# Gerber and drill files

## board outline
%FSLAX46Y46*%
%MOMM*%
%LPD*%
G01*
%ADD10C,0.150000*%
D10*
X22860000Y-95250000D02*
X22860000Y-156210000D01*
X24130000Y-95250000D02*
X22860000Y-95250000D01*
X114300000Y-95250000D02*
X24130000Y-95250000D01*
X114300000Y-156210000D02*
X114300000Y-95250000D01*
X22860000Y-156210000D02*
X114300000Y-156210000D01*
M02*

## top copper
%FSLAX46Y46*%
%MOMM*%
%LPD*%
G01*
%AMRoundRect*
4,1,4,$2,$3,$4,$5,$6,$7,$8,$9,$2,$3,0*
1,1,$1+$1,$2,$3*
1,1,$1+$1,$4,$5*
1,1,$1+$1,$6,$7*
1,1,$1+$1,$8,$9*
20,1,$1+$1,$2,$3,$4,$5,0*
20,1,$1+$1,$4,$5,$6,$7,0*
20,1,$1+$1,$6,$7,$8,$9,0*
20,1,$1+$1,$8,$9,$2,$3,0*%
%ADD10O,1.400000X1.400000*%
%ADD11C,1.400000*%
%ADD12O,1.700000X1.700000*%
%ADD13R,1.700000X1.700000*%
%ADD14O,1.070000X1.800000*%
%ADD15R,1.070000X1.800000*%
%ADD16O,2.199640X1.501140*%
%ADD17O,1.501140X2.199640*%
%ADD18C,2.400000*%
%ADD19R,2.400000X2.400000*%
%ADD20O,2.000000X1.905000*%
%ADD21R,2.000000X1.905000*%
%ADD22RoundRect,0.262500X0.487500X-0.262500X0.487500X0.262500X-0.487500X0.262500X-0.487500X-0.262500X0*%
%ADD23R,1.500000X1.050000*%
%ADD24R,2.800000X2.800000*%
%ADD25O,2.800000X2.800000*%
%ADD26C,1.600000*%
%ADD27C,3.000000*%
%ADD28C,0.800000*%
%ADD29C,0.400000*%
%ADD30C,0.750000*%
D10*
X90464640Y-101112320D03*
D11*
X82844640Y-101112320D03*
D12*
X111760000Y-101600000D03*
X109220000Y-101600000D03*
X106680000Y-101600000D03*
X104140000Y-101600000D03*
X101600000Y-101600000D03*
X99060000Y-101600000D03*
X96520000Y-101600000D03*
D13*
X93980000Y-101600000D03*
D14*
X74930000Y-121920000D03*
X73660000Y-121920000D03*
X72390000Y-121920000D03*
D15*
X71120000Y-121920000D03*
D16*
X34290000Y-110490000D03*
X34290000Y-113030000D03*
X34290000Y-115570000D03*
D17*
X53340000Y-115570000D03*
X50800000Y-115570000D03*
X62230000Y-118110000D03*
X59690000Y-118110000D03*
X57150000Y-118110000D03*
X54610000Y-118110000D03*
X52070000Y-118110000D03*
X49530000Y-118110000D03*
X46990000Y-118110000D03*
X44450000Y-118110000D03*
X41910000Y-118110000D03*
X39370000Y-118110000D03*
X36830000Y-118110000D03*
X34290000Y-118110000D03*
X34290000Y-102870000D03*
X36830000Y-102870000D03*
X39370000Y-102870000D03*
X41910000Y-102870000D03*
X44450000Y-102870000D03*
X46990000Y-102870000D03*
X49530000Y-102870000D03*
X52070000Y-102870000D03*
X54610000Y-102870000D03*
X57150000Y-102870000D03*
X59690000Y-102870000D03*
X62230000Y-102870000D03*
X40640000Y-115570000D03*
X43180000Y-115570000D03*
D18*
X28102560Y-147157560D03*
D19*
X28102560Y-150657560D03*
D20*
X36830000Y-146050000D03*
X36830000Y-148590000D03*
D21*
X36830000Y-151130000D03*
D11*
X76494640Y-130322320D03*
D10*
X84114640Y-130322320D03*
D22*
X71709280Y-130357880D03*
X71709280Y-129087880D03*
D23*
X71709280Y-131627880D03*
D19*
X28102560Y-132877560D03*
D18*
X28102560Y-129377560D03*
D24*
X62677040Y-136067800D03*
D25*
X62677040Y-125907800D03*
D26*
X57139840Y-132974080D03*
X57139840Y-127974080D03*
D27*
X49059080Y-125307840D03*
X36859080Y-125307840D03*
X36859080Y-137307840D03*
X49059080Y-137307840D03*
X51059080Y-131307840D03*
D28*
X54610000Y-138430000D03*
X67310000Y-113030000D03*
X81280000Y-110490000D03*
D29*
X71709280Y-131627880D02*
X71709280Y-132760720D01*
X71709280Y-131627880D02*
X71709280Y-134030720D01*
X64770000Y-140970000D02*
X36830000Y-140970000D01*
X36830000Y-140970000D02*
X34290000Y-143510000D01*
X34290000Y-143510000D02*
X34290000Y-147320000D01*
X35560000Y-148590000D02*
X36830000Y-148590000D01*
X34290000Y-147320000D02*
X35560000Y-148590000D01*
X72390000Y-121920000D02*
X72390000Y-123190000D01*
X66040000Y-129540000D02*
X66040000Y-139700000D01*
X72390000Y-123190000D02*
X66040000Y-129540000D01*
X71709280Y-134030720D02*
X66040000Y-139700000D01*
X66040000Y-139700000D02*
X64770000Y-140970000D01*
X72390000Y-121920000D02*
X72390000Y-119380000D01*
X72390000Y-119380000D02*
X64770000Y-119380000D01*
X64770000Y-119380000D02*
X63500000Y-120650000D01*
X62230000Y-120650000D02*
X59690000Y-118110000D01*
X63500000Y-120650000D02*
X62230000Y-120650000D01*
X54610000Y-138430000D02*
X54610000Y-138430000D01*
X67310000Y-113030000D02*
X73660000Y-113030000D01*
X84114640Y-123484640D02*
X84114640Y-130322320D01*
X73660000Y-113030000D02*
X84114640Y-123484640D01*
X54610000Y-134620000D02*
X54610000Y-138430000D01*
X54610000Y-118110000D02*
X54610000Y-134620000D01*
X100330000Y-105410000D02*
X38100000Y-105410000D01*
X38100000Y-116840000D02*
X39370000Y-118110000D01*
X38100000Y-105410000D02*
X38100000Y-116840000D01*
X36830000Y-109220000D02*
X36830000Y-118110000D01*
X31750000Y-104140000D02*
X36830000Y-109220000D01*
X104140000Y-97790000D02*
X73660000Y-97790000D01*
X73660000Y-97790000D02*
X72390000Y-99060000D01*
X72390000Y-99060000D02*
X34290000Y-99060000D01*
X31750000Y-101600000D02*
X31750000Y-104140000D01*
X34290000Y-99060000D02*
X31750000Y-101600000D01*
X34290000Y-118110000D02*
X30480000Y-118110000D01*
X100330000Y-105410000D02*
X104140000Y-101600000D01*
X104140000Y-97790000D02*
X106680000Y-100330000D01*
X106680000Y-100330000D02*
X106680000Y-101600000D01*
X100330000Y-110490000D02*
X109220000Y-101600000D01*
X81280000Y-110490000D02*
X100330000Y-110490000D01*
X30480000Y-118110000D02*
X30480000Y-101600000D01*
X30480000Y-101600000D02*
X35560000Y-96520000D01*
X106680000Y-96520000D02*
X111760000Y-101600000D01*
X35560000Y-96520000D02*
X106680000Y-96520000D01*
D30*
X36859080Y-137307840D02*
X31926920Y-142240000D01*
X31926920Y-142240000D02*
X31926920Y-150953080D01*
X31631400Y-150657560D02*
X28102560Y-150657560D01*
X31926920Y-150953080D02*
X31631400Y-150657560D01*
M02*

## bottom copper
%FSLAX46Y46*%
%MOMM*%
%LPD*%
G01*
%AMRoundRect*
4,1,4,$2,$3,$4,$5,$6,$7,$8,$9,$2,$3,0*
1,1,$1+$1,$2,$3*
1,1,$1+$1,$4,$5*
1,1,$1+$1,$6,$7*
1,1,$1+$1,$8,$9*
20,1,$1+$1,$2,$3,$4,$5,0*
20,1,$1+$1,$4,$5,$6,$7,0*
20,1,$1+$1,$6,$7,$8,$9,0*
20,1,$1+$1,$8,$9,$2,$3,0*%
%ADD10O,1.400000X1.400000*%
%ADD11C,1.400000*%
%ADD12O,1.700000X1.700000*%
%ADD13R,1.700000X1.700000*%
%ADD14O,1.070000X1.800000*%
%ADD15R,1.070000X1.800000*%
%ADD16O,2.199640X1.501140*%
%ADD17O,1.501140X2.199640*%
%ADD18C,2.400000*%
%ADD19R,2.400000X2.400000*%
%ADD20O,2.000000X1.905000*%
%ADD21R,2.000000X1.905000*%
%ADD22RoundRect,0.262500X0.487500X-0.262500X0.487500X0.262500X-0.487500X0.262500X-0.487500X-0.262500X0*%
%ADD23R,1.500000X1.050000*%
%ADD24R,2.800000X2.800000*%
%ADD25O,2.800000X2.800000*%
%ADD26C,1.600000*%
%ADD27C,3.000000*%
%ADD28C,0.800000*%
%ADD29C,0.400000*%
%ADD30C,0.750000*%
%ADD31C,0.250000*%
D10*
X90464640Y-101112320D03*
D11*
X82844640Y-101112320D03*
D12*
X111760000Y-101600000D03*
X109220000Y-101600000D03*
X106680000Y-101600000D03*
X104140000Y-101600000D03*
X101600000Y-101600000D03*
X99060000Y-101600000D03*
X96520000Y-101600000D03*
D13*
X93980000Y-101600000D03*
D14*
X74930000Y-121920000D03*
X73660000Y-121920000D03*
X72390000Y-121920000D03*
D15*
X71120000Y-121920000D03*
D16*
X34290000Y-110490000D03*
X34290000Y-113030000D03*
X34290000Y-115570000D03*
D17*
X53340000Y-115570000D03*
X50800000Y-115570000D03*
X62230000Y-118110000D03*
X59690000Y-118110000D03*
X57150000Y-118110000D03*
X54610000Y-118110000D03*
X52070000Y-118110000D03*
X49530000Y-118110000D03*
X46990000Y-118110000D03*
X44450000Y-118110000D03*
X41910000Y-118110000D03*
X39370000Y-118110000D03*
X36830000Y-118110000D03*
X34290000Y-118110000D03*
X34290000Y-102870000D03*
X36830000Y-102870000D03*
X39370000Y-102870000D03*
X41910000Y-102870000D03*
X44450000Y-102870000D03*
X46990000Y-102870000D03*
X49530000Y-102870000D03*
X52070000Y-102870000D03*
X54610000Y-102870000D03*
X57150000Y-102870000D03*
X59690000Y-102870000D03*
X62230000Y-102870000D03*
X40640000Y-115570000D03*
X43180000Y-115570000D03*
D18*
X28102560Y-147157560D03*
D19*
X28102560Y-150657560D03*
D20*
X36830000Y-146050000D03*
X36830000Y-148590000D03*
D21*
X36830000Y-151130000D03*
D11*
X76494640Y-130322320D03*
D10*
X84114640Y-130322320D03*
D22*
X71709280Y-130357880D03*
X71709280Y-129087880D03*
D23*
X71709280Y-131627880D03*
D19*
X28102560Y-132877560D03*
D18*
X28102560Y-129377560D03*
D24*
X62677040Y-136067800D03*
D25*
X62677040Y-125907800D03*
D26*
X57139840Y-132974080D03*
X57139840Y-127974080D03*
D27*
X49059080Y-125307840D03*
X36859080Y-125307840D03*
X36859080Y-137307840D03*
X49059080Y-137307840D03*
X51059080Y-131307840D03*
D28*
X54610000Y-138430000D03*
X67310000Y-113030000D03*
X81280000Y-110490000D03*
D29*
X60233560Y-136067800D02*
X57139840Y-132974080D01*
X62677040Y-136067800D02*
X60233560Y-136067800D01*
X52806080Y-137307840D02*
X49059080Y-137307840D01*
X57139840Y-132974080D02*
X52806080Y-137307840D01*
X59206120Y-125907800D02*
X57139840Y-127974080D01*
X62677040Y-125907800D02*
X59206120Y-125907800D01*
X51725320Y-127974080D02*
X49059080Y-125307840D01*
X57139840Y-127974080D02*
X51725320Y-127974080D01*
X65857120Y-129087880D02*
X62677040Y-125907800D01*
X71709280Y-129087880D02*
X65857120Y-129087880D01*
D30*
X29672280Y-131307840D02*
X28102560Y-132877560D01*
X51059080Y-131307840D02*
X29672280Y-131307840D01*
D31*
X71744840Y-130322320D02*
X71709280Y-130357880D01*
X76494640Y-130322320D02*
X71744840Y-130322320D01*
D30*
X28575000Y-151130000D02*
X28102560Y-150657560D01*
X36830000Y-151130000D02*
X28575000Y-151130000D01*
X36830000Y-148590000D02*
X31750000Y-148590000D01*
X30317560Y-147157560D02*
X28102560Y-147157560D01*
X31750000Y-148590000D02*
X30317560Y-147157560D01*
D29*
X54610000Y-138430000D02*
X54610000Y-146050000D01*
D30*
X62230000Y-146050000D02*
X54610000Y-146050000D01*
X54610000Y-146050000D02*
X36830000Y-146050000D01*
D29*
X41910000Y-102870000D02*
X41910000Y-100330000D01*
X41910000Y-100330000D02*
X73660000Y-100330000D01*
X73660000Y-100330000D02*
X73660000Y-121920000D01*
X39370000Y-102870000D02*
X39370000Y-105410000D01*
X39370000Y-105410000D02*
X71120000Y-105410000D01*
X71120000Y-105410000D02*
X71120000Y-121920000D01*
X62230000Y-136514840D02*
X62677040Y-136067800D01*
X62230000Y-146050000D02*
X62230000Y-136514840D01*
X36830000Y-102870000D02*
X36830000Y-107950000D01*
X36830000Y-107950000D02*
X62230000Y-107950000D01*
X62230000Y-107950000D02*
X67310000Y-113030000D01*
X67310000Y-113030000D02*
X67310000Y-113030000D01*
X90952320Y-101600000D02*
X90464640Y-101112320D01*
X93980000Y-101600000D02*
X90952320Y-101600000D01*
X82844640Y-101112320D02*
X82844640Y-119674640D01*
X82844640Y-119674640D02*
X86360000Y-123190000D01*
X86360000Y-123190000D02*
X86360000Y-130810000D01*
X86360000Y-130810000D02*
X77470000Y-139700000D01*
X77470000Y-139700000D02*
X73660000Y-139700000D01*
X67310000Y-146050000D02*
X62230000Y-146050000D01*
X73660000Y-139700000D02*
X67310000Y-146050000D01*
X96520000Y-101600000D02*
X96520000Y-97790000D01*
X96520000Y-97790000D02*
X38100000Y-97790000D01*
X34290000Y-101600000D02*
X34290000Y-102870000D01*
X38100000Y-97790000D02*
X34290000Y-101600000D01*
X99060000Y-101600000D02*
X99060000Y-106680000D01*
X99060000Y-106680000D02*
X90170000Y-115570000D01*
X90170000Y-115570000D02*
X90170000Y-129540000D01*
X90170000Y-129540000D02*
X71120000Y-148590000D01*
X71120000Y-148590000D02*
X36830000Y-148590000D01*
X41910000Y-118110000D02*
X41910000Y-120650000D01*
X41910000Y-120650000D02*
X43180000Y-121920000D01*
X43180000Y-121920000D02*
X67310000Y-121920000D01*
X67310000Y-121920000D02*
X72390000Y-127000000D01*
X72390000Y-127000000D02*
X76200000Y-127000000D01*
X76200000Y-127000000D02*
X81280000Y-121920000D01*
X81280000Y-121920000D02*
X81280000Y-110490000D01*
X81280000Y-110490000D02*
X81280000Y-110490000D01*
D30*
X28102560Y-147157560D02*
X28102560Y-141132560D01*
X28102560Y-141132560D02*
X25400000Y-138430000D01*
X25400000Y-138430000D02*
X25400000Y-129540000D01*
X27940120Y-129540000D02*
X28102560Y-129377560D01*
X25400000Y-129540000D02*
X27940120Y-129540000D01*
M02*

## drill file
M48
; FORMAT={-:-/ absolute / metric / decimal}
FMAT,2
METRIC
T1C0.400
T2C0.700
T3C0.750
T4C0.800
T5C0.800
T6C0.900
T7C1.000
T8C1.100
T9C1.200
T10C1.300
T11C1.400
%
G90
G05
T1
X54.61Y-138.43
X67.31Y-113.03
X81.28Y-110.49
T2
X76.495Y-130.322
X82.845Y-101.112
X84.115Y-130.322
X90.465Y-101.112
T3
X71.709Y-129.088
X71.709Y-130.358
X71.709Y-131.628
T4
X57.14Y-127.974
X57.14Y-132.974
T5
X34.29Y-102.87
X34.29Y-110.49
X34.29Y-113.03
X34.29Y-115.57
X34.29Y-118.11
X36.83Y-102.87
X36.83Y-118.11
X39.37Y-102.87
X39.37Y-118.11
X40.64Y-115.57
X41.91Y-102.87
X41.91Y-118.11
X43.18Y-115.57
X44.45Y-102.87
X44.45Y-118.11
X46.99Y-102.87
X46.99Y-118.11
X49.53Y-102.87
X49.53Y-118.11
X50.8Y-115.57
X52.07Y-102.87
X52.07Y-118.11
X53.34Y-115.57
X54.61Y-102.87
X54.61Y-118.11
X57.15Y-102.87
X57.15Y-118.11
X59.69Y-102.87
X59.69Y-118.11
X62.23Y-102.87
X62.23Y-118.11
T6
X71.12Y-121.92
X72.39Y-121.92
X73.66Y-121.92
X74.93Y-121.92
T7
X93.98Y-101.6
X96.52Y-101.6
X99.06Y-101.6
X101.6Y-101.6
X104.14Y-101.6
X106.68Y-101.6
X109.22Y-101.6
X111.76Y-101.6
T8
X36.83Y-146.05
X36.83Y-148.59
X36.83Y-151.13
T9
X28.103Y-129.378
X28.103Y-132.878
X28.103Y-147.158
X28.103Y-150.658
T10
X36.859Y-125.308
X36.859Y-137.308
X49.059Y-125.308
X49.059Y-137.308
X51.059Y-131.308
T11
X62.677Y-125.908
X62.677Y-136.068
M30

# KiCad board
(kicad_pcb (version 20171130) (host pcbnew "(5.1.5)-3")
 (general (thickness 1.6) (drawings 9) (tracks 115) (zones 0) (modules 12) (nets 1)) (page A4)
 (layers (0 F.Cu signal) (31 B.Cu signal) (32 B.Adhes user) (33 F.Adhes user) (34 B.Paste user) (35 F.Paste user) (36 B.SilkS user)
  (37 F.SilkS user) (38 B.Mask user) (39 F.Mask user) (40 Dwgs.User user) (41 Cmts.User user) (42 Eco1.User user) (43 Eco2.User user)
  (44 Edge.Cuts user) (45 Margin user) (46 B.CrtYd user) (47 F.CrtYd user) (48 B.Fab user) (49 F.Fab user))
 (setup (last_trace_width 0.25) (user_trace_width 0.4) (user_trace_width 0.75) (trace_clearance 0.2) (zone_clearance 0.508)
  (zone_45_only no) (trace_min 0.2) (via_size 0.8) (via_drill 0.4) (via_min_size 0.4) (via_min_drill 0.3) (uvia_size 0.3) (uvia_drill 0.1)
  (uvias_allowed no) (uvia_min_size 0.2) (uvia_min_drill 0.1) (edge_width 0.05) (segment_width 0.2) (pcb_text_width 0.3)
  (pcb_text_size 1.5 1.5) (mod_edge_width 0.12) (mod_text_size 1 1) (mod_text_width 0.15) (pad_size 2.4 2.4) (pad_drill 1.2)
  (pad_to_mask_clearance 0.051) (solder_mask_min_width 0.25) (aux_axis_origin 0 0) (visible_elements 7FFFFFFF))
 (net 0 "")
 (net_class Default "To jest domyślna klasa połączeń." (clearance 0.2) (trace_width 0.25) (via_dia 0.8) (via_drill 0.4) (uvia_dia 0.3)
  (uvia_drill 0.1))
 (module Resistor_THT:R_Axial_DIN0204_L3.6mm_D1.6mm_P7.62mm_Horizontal (layer F.Cu) (at 82.84464 101.11232)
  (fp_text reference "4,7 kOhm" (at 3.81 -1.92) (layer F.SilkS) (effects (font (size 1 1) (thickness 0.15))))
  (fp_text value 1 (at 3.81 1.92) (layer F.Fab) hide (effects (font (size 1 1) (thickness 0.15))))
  (pad 2 thru_hole oval (at 7.62 0) (size 1.4 1.4) (drill 0.7) (layers *.Cu *.Mask))
  (pad 1 thru_hole circle (at 0 0) (size 1.4 1.4) (drill 0.7) (layers *.Cu *.Mask)))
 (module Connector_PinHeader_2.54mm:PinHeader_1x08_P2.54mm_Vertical (layer F.Cu) (at 93.98 101.6 90)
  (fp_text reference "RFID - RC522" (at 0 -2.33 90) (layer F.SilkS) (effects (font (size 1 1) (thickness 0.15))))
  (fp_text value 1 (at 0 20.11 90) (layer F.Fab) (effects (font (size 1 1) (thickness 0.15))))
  (pad 8 thru_hole oval (at 0 17.78 90) (size 1.7 1.7) (drill 1) (layers *.Cu *.Mask))
  (pad 7 thru_hole oval (at 0 15.24 90) (size 1.7 1.7) (drill 1) (layers *.Cu *.Mask))
  (pad 6 thru_hole oval (at 0 12.7 90) (size 1.7 1.7) (drill 1) (layers *.Cu *.Mask))
  (pad 5 thru_hole oval (at 0 10.16 90) (size 1.7 1.7) (drill 1) (layers *.Cu *.Mask))
  (pad 4 thru_hole oval (at 0 7.62 90) (size 1.7 1.7) (drill 1) (layers *.Cu *.Mask))
  (pad 3 thru_hole oval (at 0 5.08 90) (size 1.7 1.7) (drill 1) (layers *.Cu *.Mask))
  (pad 2 thru_hole oval (at 0 2.54 90) (size 1.7 1.7) (drill 1) (layers *.Cu *.Mask))
  (pad 1 thru_hole rect (at 0 0 90) (size 1.7 1.7) (drill 1) (layers *.Cu *.Mask)))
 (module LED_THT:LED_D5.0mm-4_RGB (layer F.Cu) (at 71.12 121.92)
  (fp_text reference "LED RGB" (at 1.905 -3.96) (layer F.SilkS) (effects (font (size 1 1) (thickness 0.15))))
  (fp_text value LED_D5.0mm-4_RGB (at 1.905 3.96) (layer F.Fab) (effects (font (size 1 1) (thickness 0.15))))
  (pad 4 thru_hole oval (at 3.81 0) (size 1.07 1.8) (drill 0.9) (layers *.Cu *.Mask))
  (pad 3 thru_hole oval (at 2.54 0) (size 1.07 1.8) (drill 0.9) (layers *.Cu *.Mask))
  (pad 2 thru_hole oval (at 1.27 0) (size 1.07 1.8) (drill 0.9) (layers *.Cu *.Mask))
  (pad 1 thru_hole rect (at 0 0) (size 1.07 1.8) (drill 0.9) (layers *.Cu *.Mask)))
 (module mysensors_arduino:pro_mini (layer F.Cu) (at 48.26 110.49 180)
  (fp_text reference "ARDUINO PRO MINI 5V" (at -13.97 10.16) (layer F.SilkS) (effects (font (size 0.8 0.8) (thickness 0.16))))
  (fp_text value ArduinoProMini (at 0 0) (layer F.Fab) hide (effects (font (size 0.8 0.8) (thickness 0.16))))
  (pad 29 thru_hole oval (at 13.97 0 180) (size 2.19964 1.50114) (drill 0.8001) (layers *.Cu *.Mask F.SilkS))
  (pad 28 thru_hole oval (at 13.97 -2.54 180) (size 2.19964 1.50114) (drill 0.8001) (layers *.Cu *.Mask F.SilkS))
  (pad 27 thru_hole oval (at 13.97 -5.08 180) (size 2.19964 1.50114) (drill 0.8001) (layers *.Cu *.Mask F.SilkS))
  (pad 26 thru_hole oval (at -5.08 -5.08 180) (size 1.50114 2.19964) (drill 0.8001) (layers *.Cu *.Mask F.SilkS))
  (pad 25 thru_hole oval (at -2.54 -5.08 180) (size 1.50114 2.19964) (drill 0.8001) (layers *.Cu *.Mask F.SilkS))
  (pad 24 thru_hole oval (at -13.97 -7.62 180) (size 1.50114 2.19964) (drill 0.8001) (layers *.Cu *.Mask F.SilkS))
  (pad 23 thru_hole oval (at -11.43 -7.62 180) (size 1.50114 2.19964) (drill 0.8001) (layers *.Cu *.Mask F.SilkS))
  (pad 22 thru_hole oval (at -8.89 -7.62 180) (size 1.50114 2.19964) (drill 0.8001) (layers *.Cu *.Mask F.SilkS))
  (pad 21 thru_hole oval (at -6.35 -7.62 180) (size 1.50114 2.19964) (drill 0.8001) (layers *.Cu *.Mask F.SilkS))
  (pad 20 thru_hole oval (at -3.81 -7.62 180) (size 1.50114 2.19964) (drill 0.8001) (layers *.Cu *.Mask F.SilkS))
  (pad 19 thru_hole oval (at -1.27 -7.62 180) (size 1.50114 2.19964) (drill 0.8001) (layers *.Cu *.Mask F.SilkS))
  (pad 18 thru_hole oval (at 1.27 -7.62 180) (size 1.50114 2.19964) (drill 0.8001) (layers *.Cu *.Mask F.SilkS))
  (pad 17 thru_hole oval (at 3.81 -7.62 180) (size 1.50114 2.19964) (drill 0.8001) (layers *.Cu *.Mask F.SilkS))
  (pad 16 thru_hole oval (at 6.35 -7.62 180) (size 1.50114 2.19964) (drill 0.8001) (layers *.Cu *.Mask F.SilkS))
  (pad 15 thru_hole oval (at 8.89 -7.62 180) (size 1.50114 2.19964) (drill 0.8001) (layers *.Cu *.Mask F.SilkS))
  (pad 14 thru_hole oval (at 11.43 -7.62 180) (size 1.50114 2.19964) (drill 0.8001) (layers *.Cu *.Mask F.SilkS))
  (pad 13 thru_hole oval (at 13.97 -7.62 180) (size 1.50114 2.19964) (drill 0.8001) (layers *.Cu *.Mask F.SilkS))
  (pad 12 thru_hole oval (at 13.97 7.62 180) (size 1.50114 2.19964) (drill 0.8001) (layers *.Cu *.Mask F.SilkS))
  (pad 11 thru_hole oval (at 11.43 7.62 180) (size 1.50114 2.19964) (drill 0.8001) (layers *.Cu *.Mask F.SilkS))
  (pad 10 thru_hole oval (at 8.89 7.62 180) (size 1.50114 2.19964) (drill 0.8001) (layers *.Cu *.Mask F.SilkS))
  (pad 9 thru_hole oval (at 6.35 7.62 180) (size 1.50114 2.19964) (drill 0.8001) (layers *.Cu *.Mask F.SilkS))
  (pad 8 thru_hole oval (at 3.81 7.62 180) (size 1.50114 2.19964) (drill 0.8001) (layers *.Cu *.Mask F.SilkS))
  (pad 7 thru_hole oval (at 1.27 7.62 180) (size 1.50114 2.19964) (drill 0.8001) (layers *.Cu *.Mask F.SilkS))
  (pad 6 thru_hole oval (at -1.27 7.62 180) (size 1.50114 2.19964) (drill 0.8001) (layers *.Cu *.Mask F.SilkS))
  (pad 5 thru_hole oval (at -3.81 7.62 180) (size 1.50114 2.19964) (drill 0.8001) (layers *.Cu *.Mask F.SilkS))
  (pad 4 thru_hole oval (at -6.35 7.62 180) (size 1.50114 2.19964) (drill 0.8001) (layers *.Cu *.Mask F.SilkS))
  (pad 3 thru_hole oval (at -8.89 7.62 180) (size 1.50114 2.19964) (drill 0.8001) (layers *.Cu *.Mask F.SilkS))
  (pad 2 thru_hole oval (at -11.43 7.62 180) (size 1.50114 2.19964) (drill 0.8001) (layers *.Cu *.Mask F.SilkS))
  (pad 1 thru_hole oval (at -13.97 7.62 180) (size 1.50114 2.19964) (drill 0.8001) (layers *.Cu *.Mask F.SilkS))
  (pad 27 thru_hole oval (at 7.62 -5.08 180) (size 1.50114 2.19964) (drill 0.8001) (layers *.Cu *.Mask F.SilkS))
  (pad 28 thru_hole oval (at 5.08 -5.08 180) (size 1.50114 2.19964) (drill 0.8001) (layers *.Cu *.Mask F.SilkS)))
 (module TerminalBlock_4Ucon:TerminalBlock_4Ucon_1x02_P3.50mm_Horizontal (layer F.Cu) (at 28.10256 150.65756 90)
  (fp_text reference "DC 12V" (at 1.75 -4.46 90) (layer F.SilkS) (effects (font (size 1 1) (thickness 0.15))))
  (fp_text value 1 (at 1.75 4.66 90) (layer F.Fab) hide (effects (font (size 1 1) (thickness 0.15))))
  (pad 2 thru_hole circle (at 3.5 0 90) (size 2.4 2.4) (drill 1.2) (layers *.Cu *.Mask))
  (pad 1 thru_hole rect (at 0 0 90) (size 2.4 2.4) (drill 1.2) (layers *.Cu *.Mask)))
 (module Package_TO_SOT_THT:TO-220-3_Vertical (layer F.Cu) (at 36.83 151.13 90)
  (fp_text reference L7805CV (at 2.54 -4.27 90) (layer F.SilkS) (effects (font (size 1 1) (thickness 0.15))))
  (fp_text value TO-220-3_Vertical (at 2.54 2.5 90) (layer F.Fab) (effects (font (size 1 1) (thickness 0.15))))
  (pad 3 thru_hole oval (at 5.08 0 90) (size 1.905 2) (drill 1.1) (layers *.Cu *.Mask))
  (pad 2 thru_hole oval (at 2.54 0 90) (size 1.905 2) (drill 1.1) (layers *.Cu *.Mask))
  (pad 1 thru_hole rect (at 0 0 90) (size 1.905 2) (drill 1.1) (layers *.Cu *.Mask)))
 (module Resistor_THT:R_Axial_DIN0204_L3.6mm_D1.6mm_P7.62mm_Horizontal (layer F.Cu) (at 76.49464 130.32232)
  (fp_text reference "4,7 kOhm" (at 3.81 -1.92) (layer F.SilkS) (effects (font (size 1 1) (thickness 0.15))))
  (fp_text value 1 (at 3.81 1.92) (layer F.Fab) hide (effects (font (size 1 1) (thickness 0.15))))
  (pad 1 thru_hole circle (at 0 0) (size 1.4 1.4) (drill 0.7) (layers *.Cu *.Mask))
  (pad 2 thru_hole oval (at 7.62 0) (size 1.4 1.4) (drill 0.7) (layers *.Cu *.Mask)))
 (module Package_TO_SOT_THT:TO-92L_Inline (layer F.Cu) (at 71.70928 131.62788 90)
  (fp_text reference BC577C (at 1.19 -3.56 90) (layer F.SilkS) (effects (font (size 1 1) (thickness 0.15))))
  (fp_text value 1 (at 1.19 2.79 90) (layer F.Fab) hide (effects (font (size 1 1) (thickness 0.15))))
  (pad 2 thru_hole roundrect (at 1.27 0 90) (size 1.05 1.5) (drill 0.75) (layers *.Cu *.Mask) (roundrect_rratio 0.25))
  (pad 3 thru_hole roundrect (at 2.54 0 90) (size 1.05 1.5) (drill 0.75) (layers *.Cu *.Mask) (roundrect_rratio 0.25))
  (pad 1 thru_hole rect (at 0 0 90) (size 1.05 1.5) (drill 0.75) (layers *.Cu *.Mask)))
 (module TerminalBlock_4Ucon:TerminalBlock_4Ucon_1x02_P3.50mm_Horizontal (layer F.Cu) (at 28.10256 132.87756 90)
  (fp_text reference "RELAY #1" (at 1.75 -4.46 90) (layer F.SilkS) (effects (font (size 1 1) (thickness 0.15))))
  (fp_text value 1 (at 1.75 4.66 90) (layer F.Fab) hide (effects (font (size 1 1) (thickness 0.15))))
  (pad 1 thru_hole rect (at 0 0 90) (size 2.4 2.4) (drill 1.2) (layers *.Cu *.Mask))
  (pad 2 thru_hole circle (at 3.5 0 90) (size 2.4 2.4) (drill 1.2) (layers *.Cu *.Mask)))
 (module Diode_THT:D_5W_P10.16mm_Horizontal (layer F.Cu) (at 62.67704 136.0678 90)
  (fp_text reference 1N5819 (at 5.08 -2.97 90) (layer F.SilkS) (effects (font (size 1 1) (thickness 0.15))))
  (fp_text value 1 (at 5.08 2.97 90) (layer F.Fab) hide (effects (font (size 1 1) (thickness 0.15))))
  (pad 1 thru_hole rect (at 0 0 90) (size 2.8 2.8) (drill 1.4) (layers *.Cu *.Mask))
  (pad 2 thru_hole oval (at 10.16 0 90) (size 2.8 2.8) (drill 1.4) (layers *.Cu *.Mask)))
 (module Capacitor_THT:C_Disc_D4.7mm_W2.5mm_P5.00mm (layer F.Cu) (at 57.13984 132.97408 90)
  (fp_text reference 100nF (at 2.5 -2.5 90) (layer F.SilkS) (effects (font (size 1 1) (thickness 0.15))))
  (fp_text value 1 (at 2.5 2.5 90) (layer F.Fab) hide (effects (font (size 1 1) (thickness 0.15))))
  (pad 1 thru_hole circle (at 0 0 90) (size 1.6 1.6) (drill 0.8) (layers *.Cu *.Mask))
  (pad 2 thru_hole circle (at 5 0 90) (size 1.6 1.6) (drill 0.8) (layers *.Cu *.Mask)))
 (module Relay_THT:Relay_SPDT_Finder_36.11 (layer F.Cu) (at 51.05908 131.30784 180)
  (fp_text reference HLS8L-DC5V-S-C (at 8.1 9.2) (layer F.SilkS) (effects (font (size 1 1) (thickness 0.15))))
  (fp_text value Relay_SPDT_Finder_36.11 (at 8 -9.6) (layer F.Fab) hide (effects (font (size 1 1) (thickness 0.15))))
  (pad A1 thru_hole circle (at 2 6 180) (size 3 3) (drill 1.3) (layers *.Cu *.Mask))
  (pad 14 thru_hole circle (at 14.2 6 180) (size 3 3) (drill 1.3) (layers *.Cu *.Mask))
  (pad 12 thru_hole circle (at 14.2 -6 180) (size 3 3) (drill 1.3) (layers *.Cu *.Mask))
  (pad A2 thru_hole circle (at 2 -6 180) (size 3 3) (drill 1.3) (layers *.Cu *.Mask))
  (pad 11 thru_hole circle (at 0 0 180) (size 3 3) (drill 1.3) (layers *.Cu *.Mask)))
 (gr_line (start 22.86 95.25) (end 22.86 156.21) (layer Edge.Cuts) (width 0.15))
 (gr_line (start 24.13 95.25) (end 22.86 95.25) (layer Edge.Cuts) (width 0.15))
 (gr_line (start 114.3 95.25) (end 24.13 95.25) (layer Edge.Cuts) (width 0.15))
 (gr_line (start 114.3 156.21) (end 114.3 95.25) (layer Edge.Cuts) (width 0.15))
 (gr_line (start 22.86 156.21) (end 114.3 156.21) (layer Edge.Cuts) (width 0.15))
 (segment (start 60.23356 136.0678) (end 57.13984 132.97408) (width 0.4) (layer B.Cu) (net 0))
 (segment (start 62.67704 136.0678) (end 60.23356 136.0678) (width 0.4) (layer B.Cu) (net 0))
 (segment (start 52.80608 137.30784) (end 49.05908 137.30784) (width 0.4) (layer B.Cu) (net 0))
 (segment (start 57.13984 132.97408) (end 52.80608 137.30784) (width 0.4) (layer B.Cu) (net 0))
 (segment (start 59.20612 125.9078) (end 57.13984 127.97408) (width 0.4) (layer B.Cu) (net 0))
 (segment (start 62.67704 125.9078) (end 59.20612 125.9078) (width 0.4) (layer B.Cu) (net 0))
 (segment (start 51.72532 127.97408) (end 49.05908 125.30784) (width 0.4) (layer B.Cu) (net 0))
 (segment (start 57.13984 127.97408) (end 51.72532 127.97408) (width 0.4) (layer B.Cu) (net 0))
 (segment (start 65.85712 129.08788) (end 62.67704 125.9078) (width 0.4) (layer B.Cu) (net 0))
 (segment (start 71.70928 129.08788) (end 65.85712 129.08788) (width 0.4) (layer B.Cu) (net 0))
 (segment (start 29.67228 131.30784) (end 28.10256 132.87756) (width 0.75) (layer B.Cu) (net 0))
 (segment (start 51.05908 131.30784) (end 29.67228 131.30784) (width 0.75) (layer B.Cu) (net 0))
 (segment (start 71.74484 130.32232) (end 71.70928 130.35788) (width 0.25) (layer B.Cu) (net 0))
 (segment (start 76.49464 130.32232) (end 71.74484 130.32232) (width 0.25) (layer B.Cu) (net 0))
 (segment (start 71.70928 131.62788) (end 71.70928 132.76072) (width 0.4) (layer F.Cu) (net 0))
 (segment (start 28.575 151.13) (end 28.10256 150.65756) (width 0.75) (layer B.Cu) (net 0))
 (segment (start 36.83 151.13) (end 28.575 151.13) (width 0.75) (layer B.Cu) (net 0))
 (segment (start 36.83 148.59) (end 31.75 148.59) (width 0.75) (layer B.Cu) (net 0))
 (segment (start 30.31756 147.15756) (end 28.10256 147.15756) (width 0.75) (layer B.Cu) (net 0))
 (segment (start 31.75 148.59) (end 30.31756 147.15756) (width 0.75) (layer B.Cu) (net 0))
 (segment (start 71.70928 131.62788) (end 71.70928 134.03072) (width 0.4) (layer F.Cu) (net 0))
 (segment (start 64.77 140.97) (end 36.83 140.97) (width 0.4) (layer F.Cu) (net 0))
 (segment (start 36.83 140.97) (end 34.29 143.51) (width 0.4) (layer F.Cu) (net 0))
 (segment (start 34.29 143.51) (end 34.29 147.32) (width 0.4) (layer F.Cu) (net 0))
 (segment (start 35.56 148.59) (end 36.83 148.59) (width 0.4) (layer F.Cu) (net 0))
 (segment (start 34.29 147.32) (end 35.56 148.59) (width 0.4) (layer F.Cu) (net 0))
 (segment (start 72.39 121.92) (end 72.39 123.19) (width 0.4) (layer F.Cu) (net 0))
 (segment (start 66.04 129.54) (end 66.04 139.7) (width 0.4) (layer F.Cu) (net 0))
 (segment (start 72.39 123.19) (end 66.04 129.54) (width 0.4) (layer F.Cu) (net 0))
 (segment (start 71.70928 134.03072) (end 66.04 139.7) (width 0.4) (layer F.Cu) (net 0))
 (segment (start 66.04 139.7) (end 64.77 140.97) (width 0.4) (layer F.Cu) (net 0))
 (segment (start 72.39 121.92) (end 72.39 119.38) (width 0.4) (layer F.Cu) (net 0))
 (segment (start 72.39 119.38) (end 64.77 119.38) (width 0.4) (layer F.Cu) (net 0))
 (segment (start 64.77 119.38) (end 63.5 120.65) (width 0.4) (layer F.Cu) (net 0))
 (segment (start 62.23 120.65) (end 59.69 118.11) (width 0.4) (layer F.Cu) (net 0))
 (segment (start 63.5 120.65) (end 62.23 120.65) (width 0.4) (layer F.Cu) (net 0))
 (segment (start 54.61 138.43) (end 54.61 138.43) (width 0.4) (layer F.Cu) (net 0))
 (via (at 54.61 138.43) (size 0.8) (drill 0.4) (layers F.Cu B.Cu) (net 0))
 (segment (start 54.61 138.43) (end 54.61 146.05) (width 0.4) (layer B.Cu) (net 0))
 (segment (start 62.23 146.05) (end 54.61 146.05) (width 0.75) (layer B.Cu) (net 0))
 (segment (start 54.61 146.05) (end 36.83 146.05) (width 0.75) (layer B.Cu) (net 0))
 (segment (start 41.91 102.87) (end 41.91 100.33) (width 0.4) (layer B.Cu) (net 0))
 (segment (start 41.91 100.33) (end 73.66 100.33) (width 0.4) (layer B.Cu) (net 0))
 (segment (start 73.66 100.33) (end 73.66 121.92) (width 0.4) (layer B.Cu) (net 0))
 (segment (start 39.37 102.87) (end 39.37 105.41) (width 0.4) (layer B.Cu) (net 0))
 (segment (start 39.37 105.41) (end 71.12 105.41) (width 0.4) (layer B.Cu) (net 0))
 (segment (start 71.12 105.41) (end 71.12 121.92) (width 0.4) (layer B.Cu) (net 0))
 (segment (start 62.23 136.51484) (end 62.67704 136.0678) (width 0.4) (layer B.Cu) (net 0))
 (segment (start 62.23 146.05) (end 62.23 136.51484) (width 0.4) (layer B.Cu) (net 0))
 (segment (start 36.83 102.87) (end 36.83 107.95) (width 0.4) (layer B.Cu) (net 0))
 (segment (start 36.83 107.95) (end 62.23 107.95) (width 0.4) (layer B.Cu) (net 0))
 (segment (start 62.23 107.95) (end 67.31 113.03) (width 0.4) (layer B.Cu) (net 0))
 (segment (start 67.31 113.03) (end 67.31 113.03) (width 0.4) (layer B.Cu) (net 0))
 (via (at 67.31 113.03) (size 0.8) (drill 0.4) (layers F.Cu B.Cu) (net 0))
 (segment (start 67.31 113.03) (end 73.66 113.03) (width 0.4) (layer F.Cu) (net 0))
 (segment (start 84.11464 123.48464) (end 84.11464 130.32232) (width 0.4) (layer F.Cu) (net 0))
 (segment (start 73.66 113.03) (end 84.11464 123.48464) (width 0.4) (layer F.Cu) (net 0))
 (segment (start 54.61 134.62) (end 54.61 138.43) (width 0.4) (layer F.Cu) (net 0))
 (segment (start 54.61 118.11) (end 54.61 134.62) (width 0.4) (layer F.Cu) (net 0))
 (segment (start 90.95232 101.6) (end 90.46464 101.11232) (width 0.4) (layer B.Cu) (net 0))
 (segment (start 93.98 101.6) (end 90.95232 101.6) (width 0.4) (layer B.Cu) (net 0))
 (segment (start 82.84464 101.11232) (end 82.84464 119.67464) (width 0.4) (layer B.Cu) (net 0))
 (segment (start 82.84464 119.67464) (end 86.36 123.19) (width 0.4) (layer B.Cu) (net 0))
 (segment (start 86.36 123.19) (end 86.36 130.81) (width 0.4) (layer B.Cu) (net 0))
 (segment (start 86.36 130.81) (end 77.47 139.7) (width 0.4) (layer B.Cu) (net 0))
 (segment (start 77.47 139.7) (end 73.66 139.7) (width 0.4) (layer B.Cu) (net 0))
 (segment (start 67.31 146.05) (end 62.23 146.05) (width 0.4) (layer B.Cu) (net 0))
 (segment (start 73.66 139.7) (end 67.31 146.05) (width 0.4) (layer B.Cu) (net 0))
 (segment (start 96.52 101.6) (end 96.52 97.79) (width 0.4) (layer B.Cu) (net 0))
 (segment (start 96.52 97.79) (end 38.1 97.79) (width 0.4) (layer B.Cu) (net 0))
 (segment (start 34.29 101.6) (end 34.29 102.87) (width 0.4) (layer B.Cu) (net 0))
 (segment (start 38.1 97.79) (end 34.29 101.6) (width 0.4) (layer B.Cu) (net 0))
 (segment (start 99.06 101.6) (end 99.06 106.68) (width 0.4) (layer B.Cu) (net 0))
 (segment (start 99.06 106.68) (end 90.17 115.57) (width 0.4) (layer B.Cu) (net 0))
 (segment (start 90.17 115.57) (end 90.17 129.54) (width 0.4) (layer B.Cu) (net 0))
 (segment (start 90.17 129.54) (end 71.12 148.59) (width 0.4) (layer B.Cu) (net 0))
 (segment (start 71.12 148.59) (end 36.83 148.59) (width 0.4) (layer B.Cu) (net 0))
 (segment (start 100.33 105.41) (end 38.1 105.41) (width 0.4) (layer F.Cu) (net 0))
 (segment (start 38.1 116.84) (end 39.37 118.11) (width 0.4) (layer F.Cu) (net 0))
 (segment (start 38.1 105.41) (end 38.1 116.84) (width 0.4) (layer F.Cu) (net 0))
 (segment (start 36.83 109.22) (end 36.83 118.11) (width 0.4) (layer F.Cu) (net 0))
 (segment (start 31.75 104.14) (end 36.83 109.22) (width 0.4) (layer F.Cu) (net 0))
 (segment (start 104.14 97.79) (end 73.66 97.79) (width 0.4) (layer F.Cu) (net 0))
 (segment (start 73.66 97.79) (end 72.39 99.06) (width 0.4) (layer F.Cu) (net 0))
 (segment (start 72.39 99.06) (end 34.29 99.06) (width 0.4) (layer F.Cu) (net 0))
 (segment (start 31.75 101.6) (end 31.75 104.14) (width 0.4) (layer F.Cu) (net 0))
 (segment (start 34.29 99.06) (end 31.75 101.6) (width 0.4) (layer F.Cu) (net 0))
 (segment (start 34.29 118.11) (end 30.48 118.11) (width 0.4) (layer F.Cu) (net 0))
 (segment (start 41.91 118.11) (end 41.91 120.65) (width 0.4) (layer B.Cu) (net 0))
 (segment (start 41.91 120.65) (end 43.18 121.92) (width 0.4) (layer B.Cu) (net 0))
 (segment (start 43.18 121.92) (end 67.31 121.92) (width 0.4) (layer B.Cu) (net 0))
 (segment (start 67.31 121.92) (end 72.39 127) (width 0.4) (layer B.Cu) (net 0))
 (segment (start 72.39 127) (end 76.2 127) (width 0.4) (layer B.Cu) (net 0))
 (segment (start 76.2 127) (end 81.28 121.92) (width 0.4) (layer B.Cu) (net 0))
 (segment (start 81.28 121.92) (end 81.28 110.49) (width 0.4) (layer B.Cu) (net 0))
 (segment (start 100.33 105.41) (end 104.14 101.6) (width 0.4) (layer F.Cu) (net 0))
 (segment (start 104.14 97.79) (end 106.68 100.33) (width 0.4) (layer F.Cu) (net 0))
 (segment (start 106.68 100.33) (end 106.68 101.6) (width 0.4) (layer F.Cu) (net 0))
 (segment (start 81.28 110.49) (end 81.28 110.49) (width 0.4) (layer B.Cu) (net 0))
 (via (at 81.28 110.49) (size 0.8) (drill 0.4) (layers F.Cu B.Cu) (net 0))
 (segment (start 100.33 110.49) (end 109.22 101.6) (width 0.4) (layer F.Cu) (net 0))
 (segment (start 81.28 110.49) (end 100.33 110.49) (width 0.4) (layer F.Cu) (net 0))
 (segment (start 30.48 118.11) (end 30.48 101.6) (width 0.4) (layer F.Cu) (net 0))
 (segment (start 30.48 101.6) (end 35.56 96.52) (width 0.4) (layer F.Cu) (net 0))
 (segment (start 106.68 96.52) (end 111.76 101.6) (width 0.4) (layer F.Cu) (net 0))
 (segment (start 35.56 96.52) (end 106.68 96.52) (width 0.4) (layer F.Cu) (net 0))
 (segment (start 36.85908 137.30784) (end 31.92692 142.24) (width 0.75) (layer F.Cu) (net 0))
 (segment (start 31.92692 142.24) (end 31.92692 150.95308) (width 0.75) (layer F.Cu) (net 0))
 (segment (start 31.6314 150.65756) (end 28.10256 150.65756) (width 0.75) (layer F.Cu) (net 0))
 (segment (start 31.92692 150.95308) (end 31.6314 150.65756) (width 0.75) (layer F.Cu) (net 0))
 (segment (start 28.10256 147.15756) (end 28.10256 141.13256) (width 0.75) (layer B.Cu) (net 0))
 (segment (start 28.10256 141.13256) (end 25.4 138.43) (width 0.75) (layer B.Cu) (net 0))
 (segment (start 25.4 138.43) (end 25.4 129.54) (width 0.75) (layer B.Cu) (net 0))
 (segment (start 27.94012 129.54) (end 28.10256 129.37756) (width 0.75) (layer B.Cu) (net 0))
 (segment (start 25.4 129.54) (end 27.94012 129.54) (width 0.75) (layer B.Cu) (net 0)))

